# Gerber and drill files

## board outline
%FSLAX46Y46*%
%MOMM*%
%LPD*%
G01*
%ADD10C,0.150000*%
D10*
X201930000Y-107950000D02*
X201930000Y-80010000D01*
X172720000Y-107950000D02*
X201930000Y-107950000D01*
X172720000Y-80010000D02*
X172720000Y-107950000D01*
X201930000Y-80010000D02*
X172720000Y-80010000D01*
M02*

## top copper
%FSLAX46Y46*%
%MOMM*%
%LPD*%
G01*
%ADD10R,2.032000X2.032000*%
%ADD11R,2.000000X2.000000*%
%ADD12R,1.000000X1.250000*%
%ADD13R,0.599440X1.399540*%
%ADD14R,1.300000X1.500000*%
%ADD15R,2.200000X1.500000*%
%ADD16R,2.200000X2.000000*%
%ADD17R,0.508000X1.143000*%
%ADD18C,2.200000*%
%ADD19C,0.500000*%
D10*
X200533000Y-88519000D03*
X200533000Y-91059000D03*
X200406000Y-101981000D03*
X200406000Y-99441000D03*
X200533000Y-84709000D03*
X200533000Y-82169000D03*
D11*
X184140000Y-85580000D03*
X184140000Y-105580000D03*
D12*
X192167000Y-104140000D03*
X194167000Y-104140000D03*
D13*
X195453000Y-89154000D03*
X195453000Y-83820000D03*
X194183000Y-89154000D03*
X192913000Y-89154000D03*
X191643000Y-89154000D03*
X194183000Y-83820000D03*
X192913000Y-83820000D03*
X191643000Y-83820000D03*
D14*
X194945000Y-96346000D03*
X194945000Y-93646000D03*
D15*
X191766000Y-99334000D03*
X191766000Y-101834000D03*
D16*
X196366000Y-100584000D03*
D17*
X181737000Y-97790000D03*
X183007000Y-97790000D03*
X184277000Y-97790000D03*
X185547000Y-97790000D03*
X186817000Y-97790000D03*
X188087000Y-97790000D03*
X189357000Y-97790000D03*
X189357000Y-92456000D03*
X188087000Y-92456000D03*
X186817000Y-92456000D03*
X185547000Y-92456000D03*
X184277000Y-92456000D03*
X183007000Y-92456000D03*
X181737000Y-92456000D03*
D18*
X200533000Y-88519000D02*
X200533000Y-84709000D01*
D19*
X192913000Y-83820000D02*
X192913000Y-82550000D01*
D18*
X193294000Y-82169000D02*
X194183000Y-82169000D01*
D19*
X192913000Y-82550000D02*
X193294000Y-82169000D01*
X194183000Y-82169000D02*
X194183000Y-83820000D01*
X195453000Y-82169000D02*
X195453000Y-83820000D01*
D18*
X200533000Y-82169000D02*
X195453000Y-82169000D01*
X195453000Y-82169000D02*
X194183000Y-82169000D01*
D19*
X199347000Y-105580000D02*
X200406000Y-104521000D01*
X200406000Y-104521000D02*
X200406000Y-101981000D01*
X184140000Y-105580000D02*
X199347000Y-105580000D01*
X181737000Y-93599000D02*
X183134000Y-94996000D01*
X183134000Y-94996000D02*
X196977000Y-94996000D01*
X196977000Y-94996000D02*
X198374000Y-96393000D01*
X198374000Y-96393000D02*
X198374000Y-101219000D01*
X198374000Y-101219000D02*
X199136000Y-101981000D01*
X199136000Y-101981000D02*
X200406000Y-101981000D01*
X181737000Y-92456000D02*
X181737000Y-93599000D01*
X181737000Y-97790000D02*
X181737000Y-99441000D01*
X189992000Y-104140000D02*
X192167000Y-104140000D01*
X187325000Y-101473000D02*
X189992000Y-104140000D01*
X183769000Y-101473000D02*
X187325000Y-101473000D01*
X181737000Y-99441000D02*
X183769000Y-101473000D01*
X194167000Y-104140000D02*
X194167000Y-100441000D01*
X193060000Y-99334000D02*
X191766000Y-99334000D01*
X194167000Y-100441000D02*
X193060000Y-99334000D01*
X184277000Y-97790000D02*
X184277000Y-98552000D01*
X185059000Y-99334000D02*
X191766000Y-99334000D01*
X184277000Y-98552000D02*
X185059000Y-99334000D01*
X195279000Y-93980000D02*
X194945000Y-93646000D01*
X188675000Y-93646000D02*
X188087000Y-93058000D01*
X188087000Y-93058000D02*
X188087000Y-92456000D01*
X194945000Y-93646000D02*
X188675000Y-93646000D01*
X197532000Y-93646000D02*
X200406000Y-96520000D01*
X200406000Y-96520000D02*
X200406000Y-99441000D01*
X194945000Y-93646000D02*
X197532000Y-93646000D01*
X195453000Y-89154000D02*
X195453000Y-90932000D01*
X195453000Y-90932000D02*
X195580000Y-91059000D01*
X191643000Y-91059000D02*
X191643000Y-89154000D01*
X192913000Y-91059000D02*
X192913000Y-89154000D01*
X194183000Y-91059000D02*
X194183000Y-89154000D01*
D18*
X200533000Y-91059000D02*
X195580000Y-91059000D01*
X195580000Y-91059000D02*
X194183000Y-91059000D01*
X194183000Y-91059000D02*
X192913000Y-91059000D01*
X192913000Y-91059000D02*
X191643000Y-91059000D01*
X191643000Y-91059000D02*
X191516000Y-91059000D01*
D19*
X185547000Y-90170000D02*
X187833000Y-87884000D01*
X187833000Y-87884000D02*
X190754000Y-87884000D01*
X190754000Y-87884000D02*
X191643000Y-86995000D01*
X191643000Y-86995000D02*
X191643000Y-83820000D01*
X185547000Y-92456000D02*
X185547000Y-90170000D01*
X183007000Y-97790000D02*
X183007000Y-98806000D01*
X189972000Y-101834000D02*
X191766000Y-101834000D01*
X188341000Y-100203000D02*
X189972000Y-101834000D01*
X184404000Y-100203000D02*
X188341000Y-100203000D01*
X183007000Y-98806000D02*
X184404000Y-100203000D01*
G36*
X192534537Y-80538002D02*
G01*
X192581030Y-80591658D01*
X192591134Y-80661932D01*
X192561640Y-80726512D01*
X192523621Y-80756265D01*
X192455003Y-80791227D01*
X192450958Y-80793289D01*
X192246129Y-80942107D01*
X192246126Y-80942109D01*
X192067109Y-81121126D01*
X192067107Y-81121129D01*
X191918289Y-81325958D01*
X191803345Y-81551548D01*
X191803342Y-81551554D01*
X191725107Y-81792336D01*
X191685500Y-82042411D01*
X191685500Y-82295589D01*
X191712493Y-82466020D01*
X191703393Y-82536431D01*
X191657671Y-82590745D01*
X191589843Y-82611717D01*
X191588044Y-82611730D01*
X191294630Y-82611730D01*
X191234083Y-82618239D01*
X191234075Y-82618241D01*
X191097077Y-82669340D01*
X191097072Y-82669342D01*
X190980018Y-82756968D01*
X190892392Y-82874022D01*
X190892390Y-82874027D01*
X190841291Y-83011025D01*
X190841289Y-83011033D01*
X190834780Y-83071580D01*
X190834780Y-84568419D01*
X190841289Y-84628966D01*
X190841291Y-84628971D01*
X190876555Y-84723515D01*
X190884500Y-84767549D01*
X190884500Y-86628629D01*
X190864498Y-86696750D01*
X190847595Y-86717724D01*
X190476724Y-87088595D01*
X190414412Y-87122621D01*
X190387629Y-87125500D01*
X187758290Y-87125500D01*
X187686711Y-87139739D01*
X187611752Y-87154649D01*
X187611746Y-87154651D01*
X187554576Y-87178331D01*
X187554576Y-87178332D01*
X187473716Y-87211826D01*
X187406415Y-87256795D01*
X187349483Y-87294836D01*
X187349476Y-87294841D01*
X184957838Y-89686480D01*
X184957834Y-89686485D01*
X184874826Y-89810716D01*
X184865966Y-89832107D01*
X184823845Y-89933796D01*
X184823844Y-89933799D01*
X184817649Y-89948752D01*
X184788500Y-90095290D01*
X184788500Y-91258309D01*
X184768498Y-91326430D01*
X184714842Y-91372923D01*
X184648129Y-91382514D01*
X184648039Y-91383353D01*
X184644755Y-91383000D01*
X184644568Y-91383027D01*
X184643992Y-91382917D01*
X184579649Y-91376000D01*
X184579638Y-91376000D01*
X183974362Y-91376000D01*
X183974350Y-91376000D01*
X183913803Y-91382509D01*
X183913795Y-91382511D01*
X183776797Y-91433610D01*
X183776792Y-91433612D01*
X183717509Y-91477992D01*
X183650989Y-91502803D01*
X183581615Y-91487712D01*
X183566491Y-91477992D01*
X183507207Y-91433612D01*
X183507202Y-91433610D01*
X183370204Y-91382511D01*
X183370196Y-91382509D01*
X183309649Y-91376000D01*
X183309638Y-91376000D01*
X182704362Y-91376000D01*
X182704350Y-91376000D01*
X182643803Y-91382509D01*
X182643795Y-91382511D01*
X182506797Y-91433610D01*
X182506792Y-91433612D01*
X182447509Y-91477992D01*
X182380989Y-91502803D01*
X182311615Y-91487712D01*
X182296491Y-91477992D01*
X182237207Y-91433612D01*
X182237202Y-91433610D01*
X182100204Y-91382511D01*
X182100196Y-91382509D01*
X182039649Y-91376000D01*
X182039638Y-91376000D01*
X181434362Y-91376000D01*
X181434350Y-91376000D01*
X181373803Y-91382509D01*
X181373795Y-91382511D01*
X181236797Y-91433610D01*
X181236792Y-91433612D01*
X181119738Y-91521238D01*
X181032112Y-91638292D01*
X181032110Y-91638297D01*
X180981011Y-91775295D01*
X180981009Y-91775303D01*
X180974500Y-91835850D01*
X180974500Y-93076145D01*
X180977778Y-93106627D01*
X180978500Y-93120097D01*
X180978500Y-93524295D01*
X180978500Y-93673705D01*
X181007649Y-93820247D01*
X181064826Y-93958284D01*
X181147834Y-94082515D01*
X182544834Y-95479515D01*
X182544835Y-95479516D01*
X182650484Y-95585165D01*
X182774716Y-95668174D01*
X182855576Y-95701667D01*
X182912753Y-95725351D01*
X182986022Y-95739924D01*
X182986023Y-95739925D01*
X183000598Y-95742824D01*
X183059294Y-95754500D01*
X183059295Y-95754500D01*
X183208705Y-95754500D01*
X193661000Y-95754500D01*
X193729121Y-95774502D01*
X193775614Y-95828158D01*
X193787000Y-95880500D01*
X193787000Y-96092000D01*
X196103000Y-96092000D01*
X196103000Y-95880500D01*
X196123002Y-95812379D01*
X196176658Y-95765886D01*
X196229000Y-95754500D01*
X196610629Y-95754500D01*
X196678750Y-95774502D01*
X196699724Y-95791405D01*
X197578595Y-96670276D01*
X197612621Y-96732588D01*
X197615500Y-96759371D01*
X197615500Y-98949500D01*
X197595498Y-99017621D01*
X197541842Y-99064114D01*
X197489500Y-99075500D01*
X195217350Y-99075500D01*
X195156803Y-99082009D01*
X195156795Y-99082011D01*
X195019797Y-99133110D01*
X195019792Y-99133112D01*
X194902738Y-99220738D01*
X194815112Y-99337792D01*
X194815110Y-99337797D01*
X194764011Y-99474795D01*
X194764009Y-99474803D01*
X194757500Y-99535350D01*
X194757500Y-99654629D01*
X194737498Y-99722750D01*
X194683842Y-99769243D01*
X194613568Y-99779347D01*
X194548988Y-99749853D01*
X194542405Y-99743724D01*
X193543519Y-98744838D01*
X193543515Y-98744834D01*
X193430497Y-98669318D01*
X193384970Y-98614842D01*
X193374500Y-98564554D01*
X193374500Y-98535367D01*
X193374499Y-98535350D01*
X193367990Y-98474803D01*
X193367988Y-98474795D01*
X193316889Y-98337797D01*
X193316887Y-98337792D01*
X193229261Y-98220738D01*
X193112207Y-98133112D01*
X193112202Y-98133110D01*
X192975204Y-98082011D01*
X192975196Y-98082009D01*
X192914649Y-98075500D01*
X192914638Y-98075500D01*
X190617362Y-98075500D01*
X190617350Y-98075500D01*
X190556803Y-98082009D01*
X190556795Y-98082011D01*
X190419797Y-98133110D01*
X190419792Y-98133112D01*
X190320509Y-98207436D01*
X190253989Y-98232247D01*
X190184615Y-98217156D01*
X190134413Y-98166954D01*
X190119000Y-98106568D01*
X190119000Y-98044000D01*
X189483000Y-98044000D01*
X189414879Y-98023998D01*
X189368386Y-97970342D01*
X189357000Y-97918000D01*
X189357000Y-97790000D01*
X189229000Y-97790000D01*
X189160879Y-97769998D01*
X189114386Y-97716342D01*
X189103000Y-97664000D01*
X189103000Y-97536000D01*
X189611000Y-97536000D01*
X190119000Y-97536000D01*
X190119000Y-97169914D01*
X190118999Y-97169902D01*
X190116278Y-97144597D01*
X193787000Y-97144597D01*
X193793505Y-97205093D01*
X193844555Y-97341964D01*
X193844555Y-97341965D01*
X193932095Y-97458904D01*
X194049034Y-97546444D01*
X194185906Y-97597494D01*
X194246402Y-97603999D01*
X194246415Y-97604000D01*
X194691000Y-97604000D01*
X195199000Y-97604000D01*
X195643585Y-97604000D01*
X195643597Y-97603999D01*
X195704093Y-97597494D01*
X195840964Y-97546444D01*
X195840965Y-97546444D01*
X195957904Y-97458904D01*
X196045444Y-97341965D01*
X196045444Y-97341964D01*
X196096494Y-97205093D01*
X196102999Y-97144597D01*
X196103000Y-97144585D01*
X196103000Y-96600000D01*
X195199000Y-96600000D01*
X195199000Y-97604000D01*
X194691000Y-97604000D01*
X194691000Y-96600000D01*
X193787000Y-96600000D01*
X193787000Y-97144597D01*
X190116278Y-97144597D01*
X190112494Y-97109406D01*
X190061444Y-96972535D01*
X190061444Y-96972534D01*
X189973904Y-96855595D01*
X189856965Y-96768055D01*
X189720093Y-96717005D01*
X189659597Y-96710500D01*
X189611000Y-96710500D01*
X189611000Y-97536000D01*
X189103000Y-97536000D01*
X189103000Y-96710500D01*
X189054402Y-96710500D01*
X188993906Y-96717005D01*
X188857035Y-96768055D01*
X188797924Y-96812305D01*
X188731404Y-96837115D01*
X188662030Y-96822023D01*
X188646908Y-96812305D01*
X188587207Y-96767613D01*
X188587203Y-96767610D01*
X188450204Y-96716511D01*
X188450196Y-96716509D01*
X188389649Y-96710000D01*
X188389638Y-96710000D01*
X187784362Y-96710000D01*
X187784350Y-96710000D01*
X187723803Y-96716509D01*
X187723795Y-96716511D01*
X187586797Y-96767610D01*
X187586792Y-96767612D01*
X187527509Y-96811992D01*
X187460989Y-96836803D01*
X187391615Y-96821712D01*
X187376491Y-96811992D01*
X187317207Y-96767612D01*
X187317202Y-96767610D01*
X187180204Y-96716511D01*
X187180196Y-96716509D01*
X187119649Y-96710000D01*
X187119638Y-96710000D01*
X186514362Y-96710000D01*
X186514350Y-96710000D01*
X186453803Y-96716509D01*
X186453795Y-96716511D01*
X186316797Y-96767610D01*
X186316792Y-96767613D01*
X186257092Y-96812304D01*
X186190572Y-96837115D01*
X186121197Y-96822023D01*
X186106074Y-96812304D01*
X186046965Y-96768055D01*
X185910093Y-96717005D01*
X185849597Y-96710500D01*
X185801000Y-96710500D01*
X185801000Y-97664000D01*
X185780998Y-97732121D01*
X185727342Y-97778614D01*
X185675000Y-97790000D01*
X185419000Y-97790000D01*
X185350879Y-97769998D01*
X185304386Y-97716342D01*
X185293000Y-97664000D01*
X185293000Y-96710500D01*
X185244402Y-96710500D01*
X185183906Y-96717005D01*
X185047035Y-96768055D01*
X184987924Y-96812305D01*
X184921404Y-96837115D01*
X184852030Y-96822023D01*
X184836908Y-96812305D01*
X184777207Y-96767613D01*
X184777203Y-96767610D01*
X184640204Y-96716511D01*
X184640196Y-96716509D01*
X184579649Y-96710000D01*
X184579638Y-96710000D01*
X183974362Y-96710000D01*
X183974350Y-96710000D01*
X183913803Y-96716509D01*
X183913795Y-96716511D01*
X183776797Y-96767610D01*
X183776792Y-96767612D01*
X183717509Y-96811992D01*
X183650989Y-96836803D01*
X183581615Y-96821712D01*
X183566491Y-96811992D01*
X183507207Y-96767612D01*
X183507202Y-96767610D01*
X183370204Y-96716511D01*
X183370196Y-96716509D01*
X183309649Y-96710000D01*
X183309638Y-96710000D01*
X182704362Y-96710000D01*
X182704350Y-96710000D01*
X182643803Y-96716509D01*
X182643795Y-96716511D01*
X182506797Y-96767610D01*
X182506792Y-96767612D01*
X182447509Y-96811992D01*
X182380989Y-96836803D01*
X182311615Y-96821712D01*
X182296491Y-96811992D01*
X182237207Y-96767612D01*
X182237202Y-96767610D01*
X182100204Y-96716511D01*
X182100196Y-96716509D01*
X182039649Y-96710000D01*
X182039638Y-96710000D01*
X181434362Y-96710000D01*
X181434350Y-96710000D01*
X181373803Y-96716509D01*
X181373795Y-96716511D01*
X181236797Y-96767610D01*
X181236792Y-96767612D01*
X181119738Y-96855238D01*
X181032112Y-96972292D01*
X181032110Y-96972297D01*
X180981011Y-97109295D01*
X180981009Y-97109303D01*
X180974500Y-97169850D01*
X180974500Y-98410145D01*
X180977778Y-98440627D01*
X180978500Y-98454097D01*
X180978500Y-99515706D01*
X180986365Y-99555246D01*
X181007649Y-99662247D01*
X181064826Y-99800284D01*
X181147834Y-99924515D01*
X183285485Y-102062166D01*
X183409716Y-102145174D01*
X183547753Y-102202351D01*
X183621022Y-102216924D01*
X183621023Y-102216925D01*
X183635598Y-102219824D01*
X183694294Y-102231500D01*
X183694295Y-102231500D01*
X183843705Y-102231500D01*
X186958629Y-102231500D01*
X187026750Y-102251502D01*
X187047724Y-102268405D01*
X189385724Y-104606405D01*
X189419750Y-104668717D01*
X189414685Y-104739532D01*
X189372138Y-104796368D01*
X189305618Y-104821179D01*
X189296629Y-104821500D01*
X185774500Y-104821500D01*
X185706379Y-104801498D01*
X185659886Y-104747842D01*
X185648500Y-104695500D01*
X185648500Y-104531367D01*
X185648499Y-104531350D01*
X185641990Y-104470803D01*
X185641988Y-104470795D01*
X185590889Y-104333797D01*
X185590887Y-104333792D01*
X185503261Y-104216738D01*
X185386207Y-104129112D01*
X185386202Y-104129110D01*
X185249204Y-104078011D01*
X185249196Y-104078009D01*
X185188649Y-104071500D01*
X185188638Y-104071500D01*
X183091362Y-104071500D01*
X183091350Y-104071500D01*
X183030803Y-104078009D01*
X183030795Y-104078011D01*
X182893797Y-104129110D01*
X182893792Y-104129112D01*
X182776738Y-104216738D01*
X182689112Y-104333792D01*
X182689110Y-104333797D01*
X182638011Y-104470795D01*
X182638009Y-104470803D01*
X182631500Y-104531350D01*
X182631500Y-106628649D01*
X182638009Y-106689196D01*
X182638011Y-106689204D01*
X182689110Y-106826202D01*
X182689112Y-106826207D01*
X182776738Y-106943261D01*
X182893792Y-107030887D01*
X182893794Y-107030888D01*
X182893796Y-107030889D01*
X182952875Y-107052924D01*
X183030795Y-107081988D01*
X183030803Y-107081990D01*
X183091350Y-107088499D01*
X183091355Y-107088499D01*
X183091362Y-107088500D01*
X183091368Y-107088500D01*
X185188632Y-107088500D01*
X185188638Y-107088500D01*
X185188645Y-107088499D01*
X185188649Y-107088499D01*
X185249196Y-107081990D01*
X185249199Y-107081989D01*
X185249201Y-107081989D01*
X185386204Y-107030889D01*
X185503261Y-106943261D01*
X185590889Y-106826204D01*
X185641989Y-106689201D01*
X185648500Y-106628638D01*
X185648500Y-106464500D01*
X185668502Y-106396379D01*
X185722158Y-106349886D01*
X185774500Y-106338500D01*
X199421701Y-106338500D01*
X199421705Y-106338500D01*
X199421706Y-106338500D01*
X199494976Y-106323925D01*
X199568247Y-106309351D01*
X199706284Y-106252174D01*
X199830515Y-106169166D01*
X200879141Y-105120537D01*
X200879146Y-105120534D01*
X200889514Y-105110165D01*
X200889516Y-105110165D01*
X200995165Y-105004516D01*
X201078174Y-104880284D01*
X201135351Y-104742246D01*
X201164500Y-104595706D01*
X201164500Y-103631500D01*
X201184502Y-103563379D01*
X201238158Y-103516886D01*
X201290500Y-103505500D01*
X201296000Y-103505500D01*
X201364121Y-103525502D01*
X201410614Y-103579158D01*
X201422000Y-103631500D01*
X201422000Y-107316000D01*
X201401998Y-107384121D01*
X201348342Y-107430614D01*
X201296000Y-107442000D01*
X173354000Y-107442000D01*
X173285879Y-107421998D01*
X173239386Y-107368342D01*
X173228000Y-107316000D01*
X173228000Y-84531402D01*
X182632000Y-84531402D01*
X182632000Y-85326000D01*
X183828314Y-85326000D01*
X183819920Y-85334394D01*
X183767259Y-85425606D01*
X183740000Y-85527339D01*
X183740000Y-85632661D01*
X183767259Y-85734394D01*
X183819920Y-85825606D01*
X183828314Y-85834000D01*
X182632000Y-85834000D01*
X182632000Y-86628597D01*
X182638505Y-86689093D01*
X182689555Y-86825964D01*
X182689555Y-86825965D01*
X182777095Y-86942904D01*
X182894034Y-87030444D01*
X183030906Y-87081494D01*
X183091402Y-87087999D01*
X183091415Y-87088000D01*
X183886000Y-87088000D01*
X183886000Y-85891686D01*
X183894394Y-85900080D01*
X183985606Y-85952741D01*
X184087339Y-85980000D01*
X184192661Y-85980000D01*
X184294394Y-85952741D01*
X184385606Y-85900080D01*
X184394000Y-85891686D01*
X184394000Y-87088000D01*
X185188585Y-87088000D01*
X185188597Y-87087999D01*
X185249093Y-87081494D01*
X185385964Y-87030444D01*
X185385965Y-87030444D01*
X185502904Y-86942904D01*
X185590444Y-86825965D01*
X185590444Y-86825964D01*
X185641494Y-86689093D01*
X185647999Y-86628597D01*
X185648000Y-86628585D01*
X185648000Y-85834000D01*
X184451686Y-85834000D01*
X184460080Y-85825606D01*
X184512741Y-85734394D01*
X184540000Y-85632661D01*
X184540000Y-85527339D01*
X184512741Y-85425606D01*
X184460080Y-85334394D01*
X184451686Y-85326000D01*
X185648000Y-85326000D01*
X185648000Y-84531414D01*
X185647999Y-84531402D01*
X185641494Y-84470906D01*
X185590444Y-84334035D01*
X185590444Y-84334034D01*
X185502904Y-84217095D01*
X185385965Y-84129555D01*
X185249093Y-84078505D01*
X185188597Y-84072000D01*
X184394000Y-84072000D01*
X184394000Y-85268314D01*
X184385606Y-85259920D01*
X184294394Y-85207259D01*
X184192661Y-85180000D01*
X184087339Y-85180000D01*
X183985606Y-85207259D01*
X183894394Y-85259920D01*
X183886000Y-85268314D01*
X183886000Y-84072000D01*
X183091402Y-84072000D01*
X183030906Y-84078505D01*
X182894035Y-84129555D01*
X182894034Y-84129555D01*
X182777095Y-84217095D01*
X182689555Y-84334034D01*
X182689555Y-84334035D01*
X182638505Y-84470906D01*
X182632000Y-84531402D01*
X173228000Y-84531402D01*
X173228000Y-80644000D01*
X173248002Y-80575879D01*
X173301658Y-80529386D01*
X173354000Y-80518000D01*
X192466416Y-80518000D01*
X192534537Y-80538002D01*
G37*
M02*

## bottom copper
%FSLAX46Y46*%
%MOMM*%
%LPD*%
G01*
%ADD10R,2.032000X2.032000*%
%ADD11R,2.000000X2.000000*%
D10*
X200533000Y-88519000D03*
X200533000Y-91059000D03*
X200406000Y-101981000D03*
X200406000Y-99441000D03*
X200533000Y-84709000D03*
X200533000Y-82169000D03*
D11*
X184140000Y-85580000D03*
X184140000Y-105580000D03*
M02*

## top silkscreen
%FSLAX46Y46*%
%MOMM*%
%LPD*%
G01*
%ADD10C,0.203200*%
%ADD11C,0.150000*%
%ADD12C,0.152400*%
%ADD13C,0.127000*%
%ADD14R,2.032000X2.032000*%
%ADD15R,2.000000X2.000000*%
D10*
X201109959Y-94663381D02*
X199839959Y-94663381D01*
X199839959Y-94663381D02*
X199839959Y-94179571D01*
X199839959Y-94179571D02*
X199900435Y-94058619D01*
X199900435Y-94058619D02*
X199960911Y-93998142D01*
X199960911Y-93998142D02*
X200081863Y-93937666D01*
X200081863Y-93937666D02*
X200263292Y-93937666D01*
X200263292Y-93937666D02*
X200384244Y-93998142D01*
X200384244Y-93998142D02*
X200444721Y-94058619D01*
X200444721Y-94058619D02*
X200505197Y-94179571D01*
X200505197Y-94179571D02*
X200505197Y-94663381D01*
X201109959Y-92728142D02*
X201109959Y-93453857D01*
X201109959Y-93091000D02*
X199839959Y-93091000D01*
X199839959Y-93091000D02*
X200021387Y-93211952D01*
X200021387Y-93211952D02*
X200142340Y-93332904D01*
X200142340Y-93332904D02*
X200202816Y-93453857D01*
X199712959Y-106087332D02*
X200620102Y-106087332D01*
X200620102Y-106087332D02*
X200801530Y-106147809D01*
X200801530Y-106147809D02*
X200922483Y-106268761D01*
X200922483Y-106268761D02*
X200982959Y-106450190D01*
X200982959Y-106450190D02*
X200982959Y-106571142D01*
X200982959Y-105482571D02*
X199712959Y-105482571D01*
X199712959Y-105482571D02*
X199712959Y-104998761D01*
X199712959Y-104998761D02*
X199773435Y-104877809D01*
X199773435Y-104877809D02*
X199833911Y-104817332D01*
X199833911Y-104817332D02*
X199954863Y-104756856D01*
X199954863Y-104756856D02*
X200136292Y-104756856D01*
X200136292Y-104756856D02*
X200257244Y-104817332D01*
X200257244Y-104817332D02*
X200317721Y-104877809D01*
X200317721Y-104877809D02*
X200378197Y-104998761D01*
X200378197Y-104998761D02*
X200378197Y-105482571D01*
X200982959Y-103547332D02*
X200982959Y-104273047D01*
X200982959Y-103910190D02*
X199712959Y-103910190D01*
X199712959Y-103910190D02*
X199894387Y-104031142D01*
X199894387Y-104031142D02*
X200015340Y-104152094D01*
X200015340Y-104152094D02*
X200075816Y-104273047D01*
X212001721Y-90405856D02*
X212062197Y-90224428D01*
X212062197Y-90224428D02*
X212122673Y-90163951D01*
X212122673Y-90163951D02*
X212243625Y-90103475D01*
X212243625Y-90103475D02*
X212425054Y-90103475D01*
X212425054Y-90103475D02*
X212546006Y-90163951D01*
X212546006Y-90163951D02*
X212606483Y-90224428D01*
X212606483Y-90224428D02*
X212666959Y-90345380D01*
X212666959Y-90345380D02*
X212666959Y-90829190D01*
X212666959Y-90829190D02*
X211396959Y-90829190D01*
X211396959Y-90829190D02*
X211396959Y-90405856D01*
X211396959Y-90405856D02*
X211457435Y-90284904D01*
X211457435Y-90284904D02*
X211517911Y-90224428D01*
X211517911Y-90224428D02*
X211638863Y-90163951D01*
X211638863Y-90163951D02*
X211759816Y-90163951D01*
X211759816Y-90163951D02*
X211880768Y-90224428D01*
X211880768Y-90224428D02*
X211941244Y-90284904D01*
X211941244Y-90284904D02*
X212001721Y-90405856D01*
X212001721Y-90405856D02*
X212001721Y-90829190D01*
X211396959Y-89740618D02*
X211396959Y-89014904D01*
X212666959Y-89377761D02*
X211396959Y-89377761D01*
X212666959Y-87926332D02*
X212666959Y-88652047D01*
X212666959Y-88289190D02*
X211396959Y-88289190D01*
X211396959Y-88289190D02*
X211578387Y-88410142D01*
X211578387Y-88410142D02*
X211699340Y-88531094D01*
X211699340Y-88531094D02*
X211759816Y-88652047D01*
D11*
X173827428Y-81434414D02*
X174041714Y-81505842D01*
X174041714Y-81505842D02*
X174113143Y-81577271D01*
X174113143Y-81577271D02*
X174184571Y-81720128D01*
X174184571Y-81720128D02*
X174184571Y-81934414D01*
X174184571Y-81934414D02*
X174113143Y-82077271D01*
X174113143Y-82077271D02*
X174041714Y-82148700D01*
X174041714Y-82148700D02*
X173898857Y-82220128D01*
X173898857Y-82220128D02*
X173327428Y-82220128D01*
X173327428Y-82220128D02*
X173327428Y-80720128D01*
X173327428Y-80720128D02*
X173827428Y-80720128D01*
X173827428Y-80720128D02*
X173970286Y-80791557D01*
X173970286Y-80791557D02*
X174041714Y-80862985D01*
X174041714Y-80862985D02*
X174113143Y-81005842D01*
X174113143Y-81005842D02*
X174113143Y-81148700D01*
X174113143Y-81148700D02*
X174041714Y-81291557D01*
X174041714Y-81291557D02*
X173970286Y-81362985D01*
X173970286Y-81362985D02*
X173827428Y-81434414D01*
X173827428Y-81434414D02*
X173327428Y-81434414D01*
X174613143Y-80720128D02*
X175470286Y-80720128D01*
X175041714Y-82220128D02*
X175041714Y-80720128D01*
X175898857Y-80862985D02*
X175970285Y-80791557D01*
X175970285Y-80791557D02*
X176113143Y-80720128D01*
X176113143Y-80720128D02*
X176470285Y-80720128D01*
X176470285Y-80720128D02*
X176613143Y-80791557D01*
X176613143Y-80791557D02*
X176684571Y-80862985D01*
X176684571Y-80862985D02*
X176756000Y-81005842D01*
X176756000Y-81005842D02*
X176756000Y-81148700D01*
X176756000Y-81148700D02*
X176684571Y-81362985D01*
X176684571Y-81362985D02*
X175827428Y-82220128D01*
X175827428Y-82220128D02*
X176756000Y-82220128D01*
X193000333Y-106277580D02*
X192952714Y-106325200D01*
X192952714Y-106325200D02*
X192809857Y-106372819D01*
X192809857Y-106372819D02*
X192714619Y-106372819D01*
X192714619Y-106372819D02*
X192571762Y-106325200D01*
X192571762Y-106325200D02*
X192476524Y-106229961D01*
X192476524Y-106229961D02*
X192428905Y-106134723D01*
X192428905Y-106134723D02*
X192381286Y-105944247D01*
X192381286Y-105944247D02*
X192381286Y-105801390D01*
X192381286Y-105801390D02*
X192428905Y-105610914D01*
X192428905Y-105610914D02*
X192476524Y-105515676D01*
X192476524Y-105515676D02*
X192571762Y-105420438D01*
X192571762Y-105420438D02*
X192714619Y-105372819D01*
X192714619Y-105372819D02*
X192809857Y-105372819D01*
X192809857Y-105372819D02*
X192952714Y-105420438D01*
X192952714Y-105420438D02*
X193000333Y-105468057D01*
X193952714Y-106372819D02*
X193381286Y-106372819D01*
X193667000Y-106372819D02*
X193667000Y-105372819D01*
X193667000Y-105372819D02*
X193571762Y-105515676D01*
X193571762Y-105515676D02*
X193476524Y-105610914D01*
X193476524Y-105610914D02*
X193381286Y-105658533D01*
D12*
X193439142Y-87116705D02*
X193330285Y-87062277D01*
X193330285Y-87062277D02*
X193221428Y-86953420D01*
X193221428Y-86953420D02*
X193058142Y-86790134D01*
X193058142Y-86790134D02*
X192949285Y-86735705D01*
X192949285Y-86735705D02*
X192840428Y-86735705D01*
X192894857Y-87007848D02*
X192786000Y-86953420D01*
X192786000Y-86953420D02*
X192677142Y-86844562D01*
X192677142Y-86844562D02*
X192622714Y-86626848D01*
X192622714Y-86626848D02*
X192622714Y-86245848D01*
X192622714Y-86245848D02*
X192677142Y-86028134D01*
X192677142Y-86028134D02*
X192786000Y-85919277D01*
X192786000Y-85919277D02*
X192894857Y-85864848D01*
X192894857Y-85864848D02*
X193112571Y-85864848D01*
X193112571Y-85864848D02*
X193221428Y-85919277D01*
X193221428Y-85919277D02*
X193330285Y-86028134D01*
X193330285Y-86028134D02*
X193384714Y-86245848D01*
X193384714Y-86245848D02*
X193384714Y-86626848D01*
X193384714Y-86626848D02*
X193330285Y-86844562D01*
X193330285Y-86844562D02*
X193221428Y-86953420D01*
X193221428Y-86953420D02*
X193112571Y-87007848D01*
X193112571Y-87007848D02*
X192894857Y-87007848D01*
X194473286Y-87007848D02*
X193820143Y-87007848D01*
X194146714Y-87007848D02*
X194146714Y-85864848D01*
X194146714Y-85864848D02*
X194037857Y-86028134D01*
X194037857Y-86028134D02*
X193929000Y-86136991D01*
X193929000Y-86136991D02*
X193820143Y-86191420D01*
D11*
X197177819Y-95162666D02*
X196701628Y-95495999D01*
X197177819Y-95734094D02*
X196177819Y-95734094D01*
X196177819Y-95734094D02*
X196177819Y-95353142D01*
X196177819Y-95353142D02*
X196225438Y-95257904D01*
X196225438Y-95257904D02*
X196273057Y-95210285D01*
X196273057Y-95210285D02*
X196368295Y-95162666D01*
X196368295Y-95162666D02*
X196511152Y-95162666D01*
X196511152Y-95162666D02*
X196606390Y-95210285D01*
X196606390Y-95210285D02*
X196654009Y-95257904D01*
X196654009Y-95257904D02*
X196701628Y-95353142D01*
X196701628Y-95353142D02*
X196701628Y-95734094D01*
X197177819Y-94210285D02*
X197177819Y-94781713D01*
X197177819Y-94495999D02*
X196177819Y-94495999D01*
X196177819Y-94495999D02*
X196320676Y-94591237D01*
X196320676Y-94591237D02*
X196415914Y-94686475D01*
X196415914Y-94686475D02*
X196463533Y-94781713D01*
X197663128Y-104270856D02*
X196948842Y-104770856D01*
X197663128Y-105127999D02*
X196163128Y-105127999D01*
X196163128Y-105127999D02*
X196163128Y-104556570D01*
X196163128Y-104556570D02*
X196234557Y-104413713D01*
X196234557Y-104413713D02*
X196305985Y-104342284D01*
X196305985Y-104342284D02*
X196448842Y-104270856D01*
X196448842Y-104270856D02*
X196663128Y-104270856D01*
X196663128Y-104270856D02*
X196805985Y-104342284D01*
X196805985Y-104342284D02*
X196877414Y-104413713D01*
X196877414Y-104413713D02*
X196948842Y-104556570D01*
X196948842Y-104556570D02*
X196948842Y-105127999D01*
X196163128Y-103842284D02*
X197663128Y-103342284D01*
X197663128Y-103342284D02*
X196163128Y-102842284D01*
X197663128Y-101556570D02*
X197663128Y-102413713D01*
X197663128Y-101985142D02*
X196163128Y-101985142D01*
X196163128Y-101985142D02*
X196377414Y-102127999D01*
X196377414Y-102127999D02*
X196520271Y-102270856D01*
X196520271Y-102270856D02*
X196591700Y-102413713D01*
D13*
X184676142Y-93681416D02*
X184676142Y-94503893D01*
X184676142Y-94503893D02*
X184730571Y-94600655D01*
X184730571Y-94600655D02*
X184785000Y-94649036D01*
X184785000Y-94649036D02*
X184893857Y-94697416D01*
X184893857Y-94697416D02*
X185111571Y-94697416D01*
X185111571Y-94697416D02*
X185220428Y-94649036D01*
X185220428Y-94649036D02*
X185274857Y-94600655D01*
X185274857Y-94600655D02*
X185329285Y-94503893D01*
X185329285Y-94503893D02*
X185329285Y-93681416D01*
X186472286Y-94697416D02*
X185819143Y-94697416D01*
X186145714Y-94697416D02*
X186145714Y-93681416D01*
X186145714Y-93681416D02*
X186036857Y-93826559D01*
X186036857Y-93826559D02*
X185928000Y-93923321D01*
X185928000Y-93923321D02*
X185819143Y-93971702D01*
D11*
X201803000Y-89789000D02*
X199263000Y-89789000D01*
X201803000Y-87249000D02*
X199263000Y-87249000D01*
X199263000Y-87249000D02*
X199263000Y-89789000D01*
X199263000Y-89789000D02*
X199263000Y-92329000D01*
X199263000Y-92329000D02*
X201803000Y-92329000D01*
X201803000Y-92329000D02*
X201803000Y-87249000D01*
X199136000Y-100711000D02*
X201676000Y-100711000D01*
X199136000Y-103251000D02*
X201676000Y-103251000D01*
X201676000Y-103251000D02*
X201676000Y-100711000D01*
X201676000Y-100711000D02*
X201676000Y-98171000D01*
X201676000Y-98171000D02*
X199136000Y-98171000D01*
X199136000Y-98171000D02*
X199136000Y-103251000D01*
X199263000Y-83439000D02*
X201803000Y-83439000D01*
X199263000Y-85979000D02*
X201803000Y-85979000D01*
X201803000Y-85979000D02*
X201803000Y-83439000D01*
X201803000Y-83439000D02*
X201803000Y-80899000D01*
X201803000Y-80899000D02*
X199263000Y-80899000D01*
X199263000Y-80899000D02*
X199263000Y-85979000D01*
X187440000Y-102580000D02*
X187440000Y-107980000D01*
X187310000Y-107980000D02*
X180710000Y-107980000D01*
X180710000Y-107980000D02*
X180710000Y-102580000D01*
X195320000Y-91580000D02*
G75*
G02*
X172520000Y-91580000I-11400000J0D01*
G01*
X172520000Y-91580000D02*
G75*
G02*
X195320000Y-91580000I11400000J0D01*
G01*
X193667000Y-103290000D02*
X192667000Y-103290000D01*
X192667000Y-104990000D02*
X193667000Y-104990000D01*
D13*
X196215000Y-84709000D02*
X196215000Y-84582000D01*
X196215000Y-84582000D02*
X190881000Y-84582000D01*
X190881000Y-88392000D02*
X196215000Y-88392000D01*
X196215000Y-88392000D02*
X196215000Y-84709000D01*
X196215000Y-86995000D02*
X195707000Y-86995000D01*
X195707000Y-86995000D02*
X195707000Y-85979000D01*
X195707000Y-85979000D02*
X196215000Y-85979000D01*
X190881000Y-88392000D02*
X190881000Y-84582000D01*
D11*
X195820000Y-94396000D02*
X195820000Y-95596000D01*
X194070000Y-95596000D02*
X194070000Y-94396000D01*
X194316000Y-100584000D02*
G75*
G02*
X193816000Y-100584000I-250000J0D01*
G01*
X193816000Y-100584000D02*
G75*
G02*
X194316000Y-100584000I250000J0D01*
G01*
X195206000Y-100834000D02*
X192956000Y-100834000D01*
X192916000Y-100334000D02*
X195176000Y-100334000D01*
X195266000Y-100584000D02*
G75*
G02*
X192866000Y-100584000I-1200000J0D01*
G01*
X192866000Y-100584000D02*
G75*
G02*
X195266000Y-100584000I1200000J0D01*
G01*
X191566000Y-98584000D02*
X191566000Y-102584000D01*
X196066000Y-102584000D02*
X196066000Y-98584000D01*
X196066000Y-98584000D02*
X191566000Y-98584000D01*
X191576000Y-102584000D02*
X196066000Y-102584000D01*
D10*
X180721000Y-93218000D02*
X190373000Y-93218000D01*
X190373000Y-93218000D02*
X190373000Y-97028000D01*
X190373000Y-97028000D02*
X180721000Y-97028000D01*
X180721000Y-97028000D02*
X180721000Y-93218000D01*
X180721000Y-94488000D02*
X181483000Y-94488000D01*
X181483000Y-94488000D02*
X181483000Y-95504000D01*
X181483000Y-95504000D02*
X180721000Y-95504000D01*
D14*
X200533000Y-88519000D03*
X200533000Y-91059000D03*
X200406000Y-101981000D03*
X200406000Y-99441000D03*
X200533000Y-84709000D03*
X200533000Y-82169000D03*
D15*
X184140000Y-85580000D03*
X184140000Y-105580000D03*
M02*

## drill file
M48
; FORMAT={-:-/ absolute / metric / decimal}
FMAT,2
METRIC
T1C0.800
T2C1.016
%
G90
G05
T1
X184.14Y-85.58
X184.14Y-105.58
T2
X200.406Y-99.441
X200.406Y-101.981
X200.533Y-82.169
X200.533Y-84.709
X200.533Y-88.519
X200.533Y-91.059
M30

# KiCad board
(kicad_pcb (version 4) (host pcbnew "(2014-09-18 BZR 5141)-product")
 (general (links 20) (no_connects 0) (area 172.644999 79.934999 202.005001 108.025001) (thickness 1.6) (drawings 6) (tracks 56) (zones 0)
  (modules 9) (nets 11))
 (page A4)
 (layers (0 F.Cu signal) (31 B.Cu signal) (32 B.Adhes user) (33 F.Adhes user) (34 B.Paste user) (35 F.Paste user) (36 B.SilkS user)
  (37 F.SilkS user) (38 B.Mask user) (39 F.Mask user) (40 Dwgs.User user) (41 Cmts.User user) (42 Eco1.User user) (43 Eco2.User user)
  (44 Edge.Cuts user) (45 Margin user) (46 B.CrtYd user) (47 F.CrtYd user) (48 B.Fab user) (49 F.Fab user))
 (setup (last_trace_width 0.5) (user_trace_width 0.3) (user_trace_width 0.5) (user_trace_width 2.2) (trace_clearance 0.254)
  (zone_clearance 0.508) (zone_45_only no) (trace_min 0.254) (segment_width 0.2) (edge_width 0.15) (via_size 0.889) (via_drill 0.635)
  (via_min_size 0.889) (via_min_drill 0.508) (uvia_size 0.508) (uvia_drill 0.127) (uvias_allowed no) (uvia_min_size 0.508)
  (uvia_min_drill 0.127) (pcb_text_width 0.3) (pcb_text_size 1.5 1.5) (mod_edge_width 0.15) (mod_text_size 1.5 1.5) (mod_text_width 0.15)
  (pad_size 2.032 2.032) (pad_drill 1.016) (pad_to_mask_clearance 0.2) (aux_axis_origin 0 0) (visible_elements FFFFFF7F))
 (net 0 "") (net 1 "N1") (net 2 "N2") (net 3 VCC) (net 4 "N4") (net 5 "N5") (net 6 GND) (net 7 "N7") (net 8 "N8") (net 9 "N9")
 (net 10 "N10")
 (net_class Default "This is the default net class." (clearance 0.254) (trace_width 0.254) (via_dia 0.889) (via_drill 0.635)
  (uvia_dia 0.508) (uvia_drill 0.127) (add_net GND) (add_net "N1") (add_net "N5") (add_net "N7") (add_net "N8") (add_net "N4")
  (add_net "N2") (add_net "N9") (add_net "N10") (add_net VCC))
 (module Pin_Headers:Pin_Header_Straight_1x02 (layer F.Cu) (at 200.533 89.789 270)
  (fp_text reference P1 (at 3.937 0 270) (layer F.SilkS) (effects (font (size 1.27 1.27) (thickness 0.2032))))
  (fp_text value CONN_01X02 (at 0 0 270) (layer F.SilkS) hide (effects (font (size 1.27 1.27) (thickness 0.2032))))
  (fp_line (start 0 -1.27) (end 0 1.27) (layer F.SilkS) (width 0.15))
  (fp_line (start -2.54 -1.27) (end -2.54 1.27) (layer F.SilkS) (width 0.15))
  (fp_line (start -2.54 1.27) (end 0 1.27) (layer F.SilkS) (width 0.15))
  (fp_line (start 0 1.27) (end 2.54 1.27) (layer F.SilkS) (width 0.15))
  (fp_line (start 2.54 1.27) (end 2.54 -1.27) (layer F.SilkS) (width 0.15))
  (fp_line (start 2.54 -1.27) (end -2.54 -1.27) (layer F.SilkS) (width 0.15))
  (pad 1 thru_hole rect (at -1.27 0 270) (size 2.032 2.032) (drill 1.016) (layers *.Cu *.Mask F.SilkS) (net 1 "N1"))
  (pad 2 thru_hole rect (at 1.27 0 270) (size 2.032 2.032) (drill 1.016) (layers *.Cu *.Mask F.SilkS) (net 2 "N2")))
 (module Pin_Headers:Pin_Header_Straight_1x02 (layer F.Cu) (at 200.406 100.711 90)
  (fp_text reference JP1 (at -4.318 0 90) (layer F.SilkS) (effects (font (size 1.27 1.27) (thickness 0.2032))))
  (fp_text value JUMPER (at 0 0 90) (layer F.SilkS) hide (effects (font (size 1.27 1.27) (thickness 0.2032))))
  (fp_line (start 0 -1.27) (end 0 1.27) (layer F.SilkS) (width 0.15))
  (fp_line (start -2.54 -1.27) (end -2.54 1.27) (layer F.SilkS) (width 0.15))
  (fp_line (start -2.54 1.27) (end 0 1.27) (layer F.SilkS) (width 0.15))
  (fp_line (start 0 1.27) (end 2.54 1.27) (layer F.SilkS) (width 0.15))
  (fp_line (start 2.54 1.27) (end 2.54 -1.27) (layer F.SilkS) (width 0.15))
  (fp_line (start 2.54 -1.27) (end -2.54 -1.27) (layer F.SilkS) (width 0.15))
  (pad 1 thru_hole rect (at -1.27 0 90) (size 2.032 2.032) (drill 1.016) (layers *.Cu *.Mask F.SilkS) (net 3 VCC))
  (pad 2 thru_hole rect (at 1.27 0 90) (size 2.032 2.032) (drill 1.016) (layers *.Cu *.Mask F.SilkS) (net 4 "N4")))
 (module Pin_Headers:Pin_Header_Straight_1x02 (layer F.Cu) (at 200.533 83.439 90)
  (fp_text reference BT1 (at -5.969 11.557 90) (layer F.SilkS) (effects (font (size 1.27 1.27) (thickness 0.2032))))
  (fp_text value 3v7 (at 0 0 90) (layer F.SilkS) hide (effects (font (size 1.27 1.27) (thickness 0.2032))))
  (fp_line (start 0 -1.27) (end 0 1.27) (layer F.SilkS) (width 0.15))
  (fp_line (start -2.54 -1.27) (end -2.54 1.27) (layer F.SilkS) (width 0.15))
  (fp_line (start -2.54 1.27) (end 0 1.27) (layer F.SilkS) (width 0.15))
  (fp_line (start 0 1.27) (end 2.54 1.27) (layer F.SilkS) (width 0.15))
  (fp_line (start 2.54 1.27) (end 2.54 -1.27) (layer F.SilkS) (width 0.15))
  (fp_line (start 2.54 -1.27) (end -2.54 -1.27) (layer F.SilkS) (width 0.15))
  (pad 1 thru_hole rect (at -1.27 0 90) (size 2.032 2.032) (drill 1.016) (layers *.Cu *.Mask F.SilkS) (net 1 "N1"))
  (pad 2 thru_hole rect (at 1.27 0 90) (size 2.032 2.032) (drill 1.016) (layers *.Cu *.Mask F.SilkS) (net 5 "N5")))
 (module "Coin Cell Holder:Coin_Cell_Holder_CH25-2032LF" (layer F.Cu) (at 184.15 91.44)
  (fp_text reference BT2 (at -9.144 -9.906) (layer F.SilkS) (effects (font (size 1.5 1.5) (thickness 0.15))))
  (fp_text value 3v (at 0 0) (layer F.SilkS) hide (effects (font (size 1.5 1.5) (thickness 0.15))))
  (fp_line (start 3.29 11.14) (end 3.29 16.54) (layer F.SilkS) (width 0.15))
  (fp_line (start 3.16 16.54) (end -3.44 16.54) (layer F.SilkS) (width 0.15))
  (fp_line (start -3.44 16.54) (end -3.44 11.14) (layer F.SilkS) (width 0.15))
  (fp_circle (center -0.23 0.14) (end -0.23 11.54) (layer F.SilkS) (width 0.15))
  (pad 2 thru_hole rect (at -0.01 -5.86) (size 2 2) (drill 0.8) (layers *.Cu *.Mask F.SilkS) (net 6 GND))
  (pad 1 thru_hole rect (at -0.01 14.14) (size 2 2) (drill 0.8) (layers *.Cu *.Mask F.SilkS) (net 3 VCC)))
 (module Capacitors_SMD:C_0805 (layer F.Cu) (at 193.167 104.14)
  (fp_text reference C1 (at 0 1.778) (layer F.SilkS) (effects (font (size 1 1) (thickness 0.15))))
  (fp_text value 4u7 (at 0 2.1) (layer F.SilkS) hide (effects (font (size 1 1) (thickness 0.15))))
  (fp_line (start 0.5 -0.85) (end -0.5 -0.85) (layer F.SilkS) (width 0.15))
  (fp_line (start -0.5 0.85) (end 0.5 0.85) (layer F.SilkS) (width 0.15))
  (pad 1 smd rect (at -1 0) (size 1 1.25) (layers F.Cu F.Paste F.Mask) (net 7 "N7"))
  (pad 2 smd rect (at 1 0) (size 1 1.25) (layers F.Cu F.Paste F.Mask) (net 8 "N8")))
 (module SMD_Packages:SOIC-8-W (layer F.Cu) (at 193.548 86.487 180)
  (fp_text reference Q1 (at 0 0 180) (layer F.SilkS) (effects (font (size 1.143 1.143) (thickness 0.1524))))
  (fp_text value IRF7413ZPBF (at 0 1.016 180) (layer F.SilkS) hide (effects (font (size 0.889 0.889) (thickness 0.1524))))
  (fp_line (start -2.667 1.778) (end -2.667 1.905) (layer F.SilkS) (width 0.127))
  (fp_line (start -2.667 1.905) (end 2.667 1.905) (layer F.SilkS) (width 0.127))
  (fp_line (start 2.667 -1.905) (end -2.667 -1.905) (layer F.SilkS) (width 0.127))
  (fp_line (start -2.667 -1.905) (end -2.667 1.778) (layer F.SilkS) (width 0.127))
  (fp_line (start -2.667 -0.508) (end -2.159 -0.508) (layer F.SilkS) (width 0.127))
  (fp_line (start -2.159 -0.508) (end -2.159 0.508) (layer F.SilkS) (width 0.127))
  (fp_line (start -2.159 0.508) (end -2.667 0.508) (layer F.SilkS) (width 0.127))
  (fp_line (start 2.667 -1.905) (end 2.667 1.905) (layer F.SilkS) (width 0.127))
  (pad 8 smd rect (at -1.905 -2.667 180) (size 0.59944 1.39954) (layers F.Cu F.Paste F.Mask) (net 2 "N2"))
  (pad 1 smd rect (at -1.905 2.667 180) (size 0.59944 1.39954) (layers F.Cu F.Paste F.Mask) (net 5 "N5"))
  (pad 7 smd rect (at -0.635 -2.667 180) (size 0.59944 1.39954) (layers F.Cu F.Paste F.Mask) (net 2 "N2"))
  (pad 6 smd rect (at 0.635 -2.667 180) (size 0.59944 1.39954) (layers F.Cu F.Paste F.Mask) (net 2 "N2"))
  (pad 5 smd rect (at 1.905 -2.667 180) (size 0.59944 1.39954) (layers F.Cu F.Paste F.Mask) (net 2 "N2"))
  (pad 2 smd rect (at -0.635 2.667 180) (size 0.59944 1.39954) (layers F.Cu F.Paste F.Mask) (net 5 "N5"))
  (pad 3 smd rect (at 0.635 2.667 180) (size 0.59944 1.39954) (layers F.Cu F.Paste F.Mask) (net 5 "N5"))
  (pad 4 smd rect (at 1.905 2.667 180) (size 0.59944 1.39954) (layers F.Cu F.Paste F.Mask) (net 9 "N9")))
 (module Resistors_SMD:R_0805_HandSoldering (layer F.Cu) (at 194.945 94.996 90)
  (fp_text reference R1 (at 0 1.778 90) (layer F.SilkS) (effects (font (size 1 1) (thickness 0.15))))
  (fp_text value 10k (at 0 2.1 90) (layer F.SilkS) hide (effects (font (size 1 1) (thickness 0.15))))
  (fp_line (start 0.6 0.875) (end -0.6 0.875) (layer F.SilkS) (width 0.15))
  (fp_line (start -0.6 -0.875) (end 0.6 -0.875) (layer F.SilkS) (width 0.15))
  (pad 1 smd rect (at -1.35 0 90) (size 1.5 1.3) (layers F.Cu F.Paste F.Mask) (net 6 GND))
  (pad 2 smd rect (at 1.35 0 90) (size 1.5 1.3) (layers F.Cu F.Paste F.Mask) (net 4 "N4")))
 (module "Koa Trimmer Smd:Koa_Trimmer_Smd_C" (layer F.Cu) (at 194.056 100.584 270)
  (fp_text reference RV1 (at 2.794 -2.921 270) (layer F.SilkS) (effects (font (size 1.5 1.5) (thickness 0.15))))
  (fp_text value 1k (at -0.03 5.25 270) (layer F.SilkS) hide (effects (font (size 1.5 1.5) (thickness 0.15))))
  (fp_circle (center 0 -0.01) (end -0.2 0.14) (layer F.SilkS) (width 0.15))
  (fp_line (start 0.25 -1.15) (end 0.25 1.1) (layer F.SilkS) (width 0.15))
  (fp_line (start -0.25 1.14) (end -0.25 -1.12) (layer F.SilkS) (width 0.15))
  (fp_circle (center 0 -0.01) (end 0 1.19) (layer F.SilkS) (width 0.15))
  (fp_line (start -2 2.49) (end 2 2.49) (layer F.SilkS) (width 0.15))
  (fp_line (start 2 -2.01) (end -2 -2.01) (layer F.SilkS) (width 0.15))
  (fp_line (start -2 -2.01) (end -2 2.49) (layer F.SilkS) (width 0.15))
  (fp_line (start 2 2.48) (end 2 -2.01) (layer F.SilkS) (width 0.15))
  (pad 1 smd rect (at -1.25 2.29 270) (size 1.5 2.2) (layers F.Cu F.Paste F.Mask) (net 8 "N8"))
  (pad 3 smd rect (at 1.25 2.29 270) (size 1.5 2.2) (layers F.Cu F.Paste F.Mask) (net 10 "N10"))
  (pad 2 smd rect (at 0 -2.31 270) (size 2 2.2) (layers F.Cu F.Paste F.Mask)))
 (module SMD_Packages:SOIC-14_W (layer F.Cu) (at 185.547 94.996)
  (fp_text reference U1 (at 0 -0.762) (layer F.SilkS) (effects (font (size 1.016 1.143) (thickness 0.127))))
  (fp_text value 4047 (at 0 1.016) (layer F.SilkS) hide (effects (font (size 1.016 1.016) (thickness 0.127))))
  (fp_line (start -4.826 -1.778) (end 4.826 -1.778) (layer F.SilkS) (width 0.2032))
  (fp_line (start 4.826 -1.778) (end 4.826 2.032) (layer F.SilkS) (width 0.2032))
  (fp_line (start 4.826 2.032) (end -4.826 2.032) (layer F.SilkS) (width 0.2032))
  (fp_line (start -4.826 2.032) (end -4.826 -1.778) (layer F.SilkS) (width 0.2032))
  (fp_line (start -4.826 -0.508) (end -4.064 -0.508) (layer F.SilkS) (width 0.2032))
  (fp_line (start -4.064 -0.508) (end -4.064 0.508) (layer F.SilkS) (width 0.2032))
  (fp_line (start -4.064 0.508) (end -4.826 0.508) (layer F.SilkS) (width 0.2032))
  (pad 1 smd rect (at -3.81 2.794) (size 0.508 1.143) (layers F.Cu F.Paste F.Mask) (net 7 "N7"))
  (pad 2 smd rect (at -2.54 2.794) (size 0.508 1.143) (layers F.Cu F.Paste F.Mask) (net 10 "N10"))
  (pad 3 smd rect (at -1.27 2.794) (size 0.508 1.143) (layers F.Cu F.Paste F.Mask) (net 8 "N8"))
  (pad 4 smd rect (at 0 2.794) (size 0.508 1.143) (layers F.Cu F.Paste F.Mask) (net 6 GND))
  (pad 5 smd rect (at 1.27 2.794) (size 0.508 1.143) (layers F.Cu F.Paste F.Mask))
  (pad 6 smd rect (at 2.54 2.794) (size 0.508 1.143) (layers F.Cu F.Paste F.Mask))
  (pad 7 smd rect (at 3.81 2.794) (size 0.508 1.143) (layers F.Cu F.Paste F.Mask) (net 6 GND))
  (pad 8 smd rect (at 3.81 -2.54) (size 0.508 1.143) (layers F.Cu F.Paste F.Mask))
  (pad 9 smd rect (at 2.54 -2.54) (size 0.508 1.143) (layers F.Cu F.Paste F.Mask) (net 4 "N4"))
  (pad 10 smd rect (at 1.27 -2.54) (size 0.508 1.143) (layers F.Cu F.Paste F.Mask))
  (pad 11 smd rect (at 0 -2.54) (size 0.508 1.143) (layers F.Cu F.Paste F.Mask) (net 9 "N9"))
  (pad 12 smd rect (at -1.27 -2.54) (size 0.508 1.143) (layers F.Cu F.Paste F.Mask))
  (pad 13 smd rect (at -2.54 -2.54) (size 0.508 1.143) (layers F.Cu F.Paste F.Mask))
  (pad 14 smd rect (at -3.81 -2.54) (size 0.508 1.143) (layers F.Cu F.Paste F.Mask) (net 3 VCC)))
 (gr_line (start 201.93 107.95) (end 201.93 80.01) (angle 90) (layer Edge.Cuts) (width 0.15))
 (gr_line (start 172.72 107.95) (end 201.93 107.95) (angle 90) (layer Edge.Cuts) (width 0.15))
 (gr_line (start 172.72 80.01) (end 172.72 107.95) (angle 90) (layer Edge.Cuts) (width 0.15))
 (gr_line (start 201.93 80.01) (end 172.72 80.01) (angle 90) (layer Edge.Cuts) (width 0.15))
 (segment (start 200.533 88.519) (end 200.533 84.709) (width 2.2) (layer F.Cu) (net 1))
 (segment (start 192.913 83.82) (end 192.913 82.55) (width 0.5) (layer F.Cu) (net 5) (status 400000))
 (segment (start 193.294 82.169) (end 194.183 82.169) (width 2.2) (layer F.Cu) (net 5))
 (segment (start 192.913 82.55) (end 193.294 82.169) (width 0.5) (layer F.Cu) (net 5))
 (segment (start 194.183 82.169) (end 194.183 83.82) (width 0.5) (layer F.Cu) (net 5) (status 800000))
 (segment (start 195.453 82.169) (end 195.453 83.82) (width 0.5) (layer F.Cu) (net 5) (status 800000))
 (segment (start 200.533 82.169) (end 195.453 82.169) (width 2.2) (layer F.Cu) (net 5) (status 400000))
 (segment (start 195.453 82.169) (end 194.183 82.169) (width 2.2) (layer F.Cu) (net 5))
 (segment (start 199.347 105.58) (end 200.406 104.521) (width 0.5) (layer F.Cu) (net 3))
 (segment (start 200.406 104.521) (end 200.406 101.981) (width 0.5) (layer F.Cu) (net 3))
 (segment (start 184.14 105.58) (end 199.347 105.58) (width 0.5) (layer F.Cu) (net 3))
 (segment (start 181.737 93.599) (end 183.134 94.996) (width 0.5) (layer F.Cu) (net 3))
 (segment (start 183.134 94.996) (end 196.977 94.996) (width 0.5) (layer F.Cu) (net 3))
 (segment (start 196.977 94.996) (end 198.374 96.393) (width 0.5) (layer F.Cu) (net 3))
 (segment (start 198.374 96.393) (end 198.374 101.219) (width 0.5) (layer F.Cu) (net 3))
 (segment (start 198.374 101.219) (end 199.136 101.981) (width 0.5) (layer F.Cu) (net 3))
 (segment (start 199.136 101.981) (end 200.406 101.981) (width 0.5) (layer F.Cu) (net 3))
 (segment (start 181.737 92.456) (end 181.737 93.599) (width 0.5) (layer F.Cu) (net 3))
 (segment (start 181.737 97.79) (end 181.737 99.441) (width 0.5) (layer F.Cu) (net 7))
 (segment (start 189.992 104.14) (end 192.167 104.14) (width 0.5) (layer F.Cu) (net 7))
 (segment (start 187.325 101.473) (end 189.992 104.14) (width 0.5) (layer F.Cu) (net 7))
 (segment (start 183.769 101.473) (end 187.325 101.473) (width 0.5) (layer F.Cu) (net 7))
 (segment (start 181.737 99.441) (end 183.769 101.473) (width 0.5) (layer F.Cu) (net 7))
 (segment (start 194.167 104.14) (end 194.167 100.441) (width 0.5) (layer F.Cu) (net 8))
 (segment (start 193.06 99.334) (end 191.766 99.334) (width 0.5) (layer F.Cu) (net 8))
 (segment (start 194.167 100.441) (end 193.06 99.334) (width 0.5) (layer F.Cu) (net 8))
 (segment (start 184.277 97.79) (end 184.277 98.552) (width 0.5) (layer F.Cu) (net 8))
 (segment (start 185.059 99.334) (end 191.766 99.334) (width 0.5) (layer F.Cu) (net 8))
 (segment (start 184.277 98.552) (end 185.059 99.334) (width 0.5) (layer F.Cu) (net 8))
 (segment (start 195.279 93.98) (end 194.945 93.646) (width 0.5) (layer F.Cu) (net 4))
 (segment (start 188.675 93.646) (end 188.087 93.058) (width 0.5) (layer F.Cu) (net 4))
 (segment (start 188.087 93.058) (end 188.087 92.456) (width 0.5) (layer F.Cu) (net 4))
 (segment (start 194.945 93.646) (end 188.675 93.646) (width 0.5) (layer F.Cu) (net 4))
 (segment (start 197.532 93.646) (end 200.406 96.52) (width 0.5) (layer F.Cu) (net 4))
 (segment (start 200.406 96.52) (end 200.406 99.441) (width 0.5) (layer F.Cu) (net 4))
 (segment (start 194.945 93.646) (end 197.532 93.646) (width 0.5) (layer F.Cu) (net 4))
 (segment (start 195.453 89.154) (end 195.453 90.932) (width 0.5) (layer F.Cu) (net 2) (status 400000))
 (segment (start 195.453 90.932) (end 195.58 91.059) (width 0.5) (layer F.Cu) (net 2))
 (segment (start 191.643 91.059) (end 191.643 89.154) (width 0.5) (layer F.Cu) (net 2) (status 800000))
 (segment (start 192.913 91.059) (end 192.913 89.154) (width 0.5) (layer F.Cu) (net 2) (status 800000))
 (segment (start 194.183 91.059) (end 194.183 89.154) (width 0.5) (layer F.Cu) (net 2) (status 800000))
 (segment (start 200.533 91.059) (end 195.58 91.059) (width 2.2) (layer F.Cu) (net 2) (status 400000))
 (segment (start 195.58 91.059) (end 194.183 91.059) (width 2.2) (layer F.Cu) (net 2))
 (segment (start 194.183 91.059) (end 192.913 91.059) (width 2.2) (layer F.Cu) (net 2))
 (segment (start 192.913 91.059) (end 191.643 91.059) (width 2.2) (layer F.Cu) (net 2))
 (segment (start 191.643 91.059) (end 191.516 91.059) (width 2.2) (layer F.Cu) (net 2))
 (segment (start 185.547 90.17) (end 187.833 87.884) (width 0.5) (layer F.Cu) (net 9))
 (segment (start 187.833 87.884) (end 190.754 87.884) (width 0.5) (layer F.Cu) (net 9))
 (segment (start 190.754 87.884) (end 191.643 86.995) (width 0.5) (layer F.Cu) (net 9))
 (segment (start 191.643 86.995) (end 191.643 83.82) (width 0.5) (layer F.Cu) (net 9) (status 20))
 (segment (start 185.547 92.456) (end 185.547 90.17) (width 0.5) (layer F.Cu) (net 9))
 (segment (start 183.007 97.79) (end 183.007 98.806) (width 0.5) (layer F.Cu) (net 10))
 (segment (start 189.972 101.834) (end 191.766 101.834) (width 0.5) (layer F.Cu) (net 10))
 (segment (start 188.341 100.203) (end 189.972 101.834) (width 0.5) (layer F.Cu) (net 10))
 (segment (start 184.404 100.203) (end 188.341 100.203) (width 0.5) (layer F.Cu) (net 10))
 (segment (start 183.007 98.806) (end 184.404 100.203) (width 0.5) (layer F.Cu) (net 10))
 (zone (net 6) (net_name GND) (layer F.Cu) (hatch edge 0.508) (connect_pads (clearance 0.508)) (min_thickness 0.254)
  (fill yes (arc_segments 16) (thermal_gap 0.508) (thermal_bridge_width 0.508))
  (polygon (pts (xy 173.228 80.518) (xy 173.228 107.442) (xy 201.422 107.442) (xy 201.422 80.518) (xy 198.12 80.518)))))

